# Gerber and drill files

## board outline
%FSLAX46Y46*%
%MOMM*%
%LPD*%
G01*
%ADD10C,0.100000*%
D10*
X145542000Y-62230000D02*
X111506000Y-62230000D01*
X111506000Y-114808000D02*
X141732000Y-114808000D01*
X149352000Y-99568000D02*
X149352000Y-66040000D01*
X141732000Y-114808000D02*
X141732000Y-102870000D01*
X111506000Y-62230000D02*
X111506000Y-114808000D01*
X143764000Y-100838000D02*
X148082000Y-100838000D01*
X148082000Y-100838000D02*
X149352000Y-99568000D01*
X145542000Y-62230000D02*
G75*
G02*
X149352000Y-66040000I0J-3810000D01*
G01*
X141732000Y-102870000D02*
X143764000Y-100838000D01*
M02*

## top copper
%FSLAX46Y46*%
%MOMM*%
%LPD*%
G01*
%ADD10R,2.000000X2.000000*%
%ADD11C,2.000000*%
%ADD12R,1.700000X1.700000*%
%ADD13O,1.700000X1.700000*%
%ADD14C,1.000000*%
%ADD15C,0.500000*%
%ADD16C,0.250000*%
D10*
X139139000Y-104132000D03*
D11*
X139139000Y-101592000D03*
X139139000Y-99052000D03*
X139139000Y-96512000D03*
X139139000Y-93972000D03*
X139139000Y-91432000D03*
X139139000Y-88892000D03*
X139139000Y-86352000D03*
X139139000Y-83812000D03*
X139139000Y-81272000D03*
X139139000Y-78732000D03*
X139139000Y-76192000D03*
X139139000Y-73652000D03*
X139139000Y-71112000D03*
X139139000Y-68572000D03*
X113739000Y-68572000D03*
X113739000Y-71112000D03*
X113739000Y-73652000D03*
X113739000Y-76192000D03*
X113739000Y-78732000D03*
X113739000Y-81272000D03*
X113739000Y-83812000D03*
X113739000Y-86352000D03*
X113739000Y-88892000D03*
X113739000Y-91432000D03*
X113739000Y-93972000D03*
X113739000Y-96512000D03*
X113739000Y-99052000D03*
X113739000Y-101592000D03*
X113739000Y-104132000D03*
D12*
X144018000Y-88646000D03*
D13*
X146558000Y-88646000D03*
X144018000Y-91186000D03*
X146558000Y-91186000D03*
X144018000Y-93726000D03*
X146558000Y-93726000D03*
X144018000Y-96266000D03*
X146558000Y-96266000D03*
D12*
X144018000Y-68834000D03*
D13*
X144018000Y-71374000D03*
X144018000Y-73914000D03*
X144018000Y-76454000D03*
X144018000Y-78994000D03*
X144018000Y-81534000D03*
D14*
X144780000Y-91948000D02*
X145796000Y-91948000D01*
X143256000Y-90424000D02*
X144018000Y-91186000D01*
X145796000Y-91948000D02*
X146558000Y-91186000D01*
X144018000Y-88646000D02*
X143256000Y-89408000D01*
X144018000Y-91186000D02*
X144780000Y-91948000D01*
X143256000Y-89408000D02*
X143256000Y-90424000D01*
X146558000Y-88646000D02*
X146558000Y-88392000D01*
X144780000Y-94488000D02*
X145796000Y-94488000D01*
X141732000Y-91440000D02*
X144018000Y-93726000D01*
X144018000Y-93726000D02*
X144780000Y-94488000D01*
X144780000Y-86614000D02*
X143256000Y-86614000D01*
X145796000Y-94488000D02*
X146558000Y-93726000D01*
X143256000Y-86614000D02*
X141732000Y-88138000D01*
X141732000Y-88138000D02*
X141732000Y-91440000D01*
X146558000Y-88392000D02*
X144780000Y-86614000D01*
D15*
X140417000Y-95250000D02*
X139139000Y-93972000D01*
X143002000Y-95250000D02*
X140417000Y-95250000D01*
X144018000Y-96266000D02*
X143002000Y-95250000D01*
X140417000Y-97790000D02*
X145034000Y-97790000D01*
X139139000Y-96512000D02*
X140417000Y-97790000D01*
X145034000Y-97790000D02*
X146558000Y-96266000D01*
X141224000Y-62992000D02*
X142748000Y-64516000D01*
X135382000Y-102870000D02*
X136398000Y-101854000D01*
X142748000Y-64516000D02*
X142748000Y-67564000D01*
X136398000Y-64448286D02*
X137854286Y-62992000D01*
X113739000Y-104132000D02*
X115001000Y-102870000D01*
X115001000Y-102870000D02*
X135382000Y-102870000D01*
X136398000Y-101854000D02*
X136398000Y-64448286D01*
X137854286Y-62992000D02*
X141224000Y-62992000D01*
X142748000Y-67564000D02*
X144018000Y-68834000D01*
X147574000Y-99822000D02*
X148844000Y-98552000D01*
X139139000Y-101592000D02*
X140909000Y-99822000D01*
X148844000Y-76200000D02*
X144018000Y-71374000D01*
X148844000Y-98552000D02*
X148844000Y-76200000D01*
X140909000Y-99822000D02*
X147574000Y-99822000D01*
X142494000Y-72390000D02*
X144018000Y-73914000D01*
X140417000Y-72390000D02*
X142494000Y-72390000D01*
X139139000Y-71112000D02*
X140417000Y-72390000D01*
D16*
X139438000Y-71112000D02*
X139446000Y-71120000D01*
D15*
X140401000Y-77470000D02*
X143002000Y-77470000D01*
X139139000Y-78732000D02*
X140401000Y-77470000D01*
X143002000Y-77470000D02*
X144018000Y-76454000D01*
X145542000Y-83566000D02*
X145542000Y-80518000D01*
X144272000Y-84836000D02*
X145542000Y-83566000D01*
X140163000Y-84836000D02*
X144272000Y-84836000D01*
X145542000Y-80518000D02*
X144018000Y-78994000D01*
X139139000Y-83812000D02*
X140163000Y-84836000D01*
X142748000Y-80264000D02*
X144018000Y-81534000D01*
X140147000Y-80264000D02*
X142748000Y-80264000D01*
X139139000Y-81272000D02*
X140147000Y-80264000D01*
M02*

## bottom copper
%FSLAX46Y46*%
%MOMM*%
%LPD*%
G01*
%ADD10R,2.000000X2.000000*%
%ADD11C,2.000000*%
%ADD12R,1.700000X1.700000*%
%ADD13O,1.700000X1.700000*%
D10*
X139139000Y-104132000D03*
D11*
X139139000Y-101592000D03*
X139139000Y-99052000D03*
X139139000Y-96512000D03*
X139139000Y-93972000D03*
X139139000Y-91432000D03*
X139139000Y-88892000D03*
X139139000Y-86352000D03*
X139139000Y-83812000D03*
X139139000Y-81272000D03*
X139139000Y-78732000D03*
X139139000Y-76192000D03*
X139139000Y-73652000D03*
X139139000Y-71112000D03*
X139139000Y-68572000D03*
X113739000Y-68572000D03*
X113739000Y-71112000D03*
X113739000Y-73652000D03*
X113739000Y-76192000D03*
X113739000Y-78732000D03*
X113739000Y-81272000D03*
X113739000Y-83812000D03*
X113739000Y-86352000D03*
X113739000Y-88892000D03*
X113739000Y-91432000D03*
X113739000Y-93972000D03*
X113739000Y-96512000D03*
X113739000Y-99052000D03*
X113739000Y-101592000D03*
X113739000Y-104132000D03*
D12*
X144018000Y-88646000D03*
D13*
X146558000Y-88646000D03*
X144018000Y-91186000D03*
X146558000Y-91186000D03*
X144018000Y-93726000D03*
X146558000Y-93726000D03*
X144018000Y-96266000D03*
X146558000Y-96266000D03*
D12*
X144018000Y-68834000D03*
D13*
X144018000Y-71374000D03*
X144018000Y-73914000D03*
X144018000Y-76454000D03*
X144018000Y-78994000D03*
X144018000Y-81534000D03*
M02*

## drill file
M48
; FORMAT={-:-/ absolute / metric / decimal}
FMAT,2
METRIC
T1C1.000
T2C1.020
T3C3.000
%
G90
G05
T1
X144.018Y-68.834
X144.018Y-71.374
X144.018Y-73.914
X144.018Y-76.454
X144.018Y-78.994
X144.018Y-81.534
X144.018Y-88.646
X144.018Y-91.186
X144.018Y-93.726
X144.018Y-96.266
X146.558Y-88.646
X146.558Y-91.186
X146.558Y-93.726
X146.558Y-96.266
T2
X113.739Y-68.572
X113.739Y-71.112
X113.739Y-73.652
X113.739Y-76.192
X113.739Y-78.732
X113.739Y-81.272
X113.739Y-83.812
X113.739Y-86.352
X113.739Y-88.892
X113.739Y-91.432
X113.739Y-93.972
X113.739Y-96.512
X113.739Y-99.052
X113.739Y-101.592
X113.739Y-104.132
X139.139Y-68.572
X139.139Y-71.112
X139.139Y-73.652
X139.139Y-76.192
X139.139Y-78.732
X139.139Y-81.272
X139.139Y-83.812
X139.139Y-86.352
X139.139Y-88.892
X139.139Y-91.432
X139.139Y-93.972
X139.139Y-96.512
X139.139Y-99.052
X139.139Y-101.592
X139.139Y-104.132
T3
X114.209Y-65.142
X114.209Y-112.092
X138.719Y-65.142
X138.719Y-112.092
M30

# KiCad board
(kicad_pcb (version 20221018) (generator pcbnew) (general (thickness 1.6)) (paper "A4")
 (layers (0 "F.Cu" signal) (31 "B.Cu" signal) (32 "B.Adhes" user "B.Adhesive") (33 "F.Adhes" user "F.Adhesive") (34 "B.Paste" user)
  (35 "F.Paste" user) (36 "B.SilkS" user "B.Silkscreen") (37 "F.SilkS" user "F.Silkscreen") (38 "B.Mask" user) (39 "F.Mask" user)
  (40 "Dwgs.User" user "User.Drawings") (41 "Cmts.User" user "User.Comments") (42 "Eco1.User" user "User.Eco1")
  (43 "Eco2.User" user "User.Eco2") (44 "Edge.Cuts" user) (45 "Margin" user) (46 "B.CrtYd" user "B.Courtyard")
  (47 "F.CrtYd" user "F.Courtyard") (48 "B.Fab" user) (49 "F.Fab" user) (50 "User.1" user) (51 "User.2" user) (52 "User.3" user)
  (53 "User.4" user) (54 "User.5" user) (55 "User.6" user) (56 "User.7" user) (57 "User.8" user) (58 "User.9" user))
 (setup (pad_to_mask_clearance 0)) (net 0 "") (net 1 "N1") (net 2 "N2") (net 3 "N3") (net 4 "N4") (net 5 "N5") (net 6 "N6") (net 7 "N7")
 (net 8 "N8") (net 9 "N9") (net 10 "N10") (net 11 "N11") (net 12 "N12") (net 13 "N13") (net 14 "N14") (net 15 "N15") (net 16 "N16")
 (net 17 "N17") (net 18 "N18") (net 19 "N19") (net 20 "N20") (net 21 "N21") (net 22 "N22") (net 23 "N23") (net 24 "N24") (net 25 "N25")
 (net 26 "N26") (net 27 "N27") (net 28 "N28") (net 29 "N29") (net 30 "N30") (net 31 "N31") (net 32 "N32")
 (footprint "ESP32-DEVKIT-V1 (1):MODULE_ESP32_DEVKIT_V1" (layer "F.Cu") (at 126.439 88.617 180)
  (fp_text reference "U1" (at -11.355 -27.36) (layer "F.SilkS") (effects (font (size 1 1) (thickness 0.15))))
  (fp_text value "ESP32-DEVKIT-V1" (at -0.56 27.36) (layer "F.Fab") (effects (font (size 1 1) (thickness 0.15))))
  (pad "" np_thru_hole circle (at -12.28 -23.475 180) (size 3 3) (drill 3) (layers "*.Cu" "*.Mask"))
  (pad "" np_thru_hole circle (at -12.28 23.475 180) (size 3 3) (drill 3) (layers "*.Cu" "*.Mask"))
  (pad "" np_thru_hole circle (at 12.23 -23.475 180) (size 3 3) (drill 3) (layers "*.Cu" "*.Mask"))
  (pad "" np_thru_hole circle (at 12.23 23.475 180) (size 3 3) (drill 3) (layers "*.Cu" "*.Mask"))
  (pad "1" thru_hole rect (at -12.7 -15.515 180) (size 2 2) (drill 1.02) (layers "*.Cu" "*.Mask") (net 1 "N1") (solder_mask_margin 0.102))
  (pad "2" thru_hole circle (at -12.7 -12.975 180) (size 2 2) (drill 1.02) (layers "*.Cu" "*.Mask") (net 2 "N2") (solder_mask_margin 0.102))
  (pad "3" thru_hole circle (at -12.7 -10.435 180) (size 2 2) (drill 1.02) (layers "*.Cu" "*.Mask") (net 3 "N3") (solder_mask_margin 0.102))
  (pad "4" thru_hole circle (at -12.7 -7.895 180) (size 2 2) (drill 1.02) (layers "*.Cu" "*.Mask") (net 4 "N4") (solder_mask_margin 0.102))
  (pad "5" thru_hole circle (at -12.7 -5.355 180) (size 2 2) (drill 1.02) (layers "*.Cu" "*.Mask") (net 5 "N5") (solder_mask_margin 0.102))
  (pad "6" thru_hole circle (at -12.7 -2.815 180) (size 2 2) (drill 1.02) (layers "*.Cu" "*.Mask") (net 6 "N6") (solder_mask_margin 0.102))
  (pad "7" thru_hole circle (at -12.7 -0.275 180) (size 2 2) (drill 1.02) (layers "*.Cu" "*.Mask") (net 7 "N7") (solder_mask_margin 0.102))
  (pad "8" thru_hole circle (at -12.7 2.265 180) (size 2 2) (drill 1.02) (layers "*.Cu" "*.Mask") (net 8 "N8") (solder_mask_margin 0.102))
  (pad "9" thru_hole circle (at -12.7 4.805 180) (size 2 2) (drill 1.02) (layers "*.Cu" "*.Mask") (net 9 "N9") (solder_mask_margin 0.102))
  (pad "10" thru_hole circle (at -12.7 7.345 180) (size 2 2) (drill 1.02) (layers "*.Cu" "*.Mask") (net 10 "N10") (solder_mask_margin 0.102))
  (pad "11" thru_hole circle (at -12.7 9.885 180) (size 2 2) (drill 1.02) (layers "*.Cu" "*.Mask") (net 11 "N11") (solder_mask_margin 0.102))
  (pad "12" thru_hole circle (at -12.7 12.425 180) (size 2 2) (drill 1.02) (layers "*.Cu" "*.Mask") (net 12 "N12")
   (solder_mask_margin 0.102))
  (pad "13" thru_hole circle (at -12.7 14.965 180) (size 2 2) (drill 1.02) (layers "*.Cu" "*.Mask") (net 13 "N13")
   (solder_mask_margin 0.102))
  (pad "14" thru_hole circle (at -12.7 17.505 180) (size 2 2) (drill 1.02) (layers "*.Cu" "*.Mask") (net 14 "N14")
   (solder_mask_margin 0.102))
  (pad "15" thru_hole circle (at -12.7 20.045 180) (size 2 2) (drill 1.02) (layers "*.Cu" "*.Mask") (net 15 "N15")
   (solder_mask_margin 0.102))
  (pad "16" thru_hole circle (at 12.7 20.045 180) (size 2 2) (drill 1.02) (layers "*.Cu" "*.Mask") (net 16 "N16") (solder_mask_margin 0.102))
  (pad "17" thru_hole circle (at 12.7 17.505 180) (size 2 2) (drill 1.02) (layers "*.Cu" "*.Mask") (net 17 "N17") (solder_mask_margin 0.102))
  (pad "18" thru_hole circle (at 12.7 14.965 180) (size 2 2) (drill 1.02) (layers "*.Cu" "*.Mask") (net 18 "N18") (solder_mask_margin 0.102))
  (pad "19" thru_hole circle (at 12.7 12.425 180) (size 2 2) (drill 1.02) (layers "*.Cu" "*.Mask") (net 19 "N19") (solder_mask_margin 0.102))
  (pad "20" thru_hole circle (at 12.7 9.885 180) (size 2 2) (drill 1.02) (layers "*.Cu" "*.Mask") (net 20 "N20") (solder_mask_margin 0.102))
  (pad "21" thru_hole circle (at 12.7 7.345 180) (size 2 2) (drill 1.02) (layers "*.Cu" "*.Mask") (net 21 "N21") (solder_mask_margin 0.102))
  (pad "22" thru_hole circle (at 12.7 4.805 180) (size 2 2) (drill 1.02) (layers "*.Cu" "*.Mask") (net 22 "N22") (solder_mask_margin 0.102))
  (pad "23" thru_hole circle (at 12.7 2.265 180) (size 2 2) (drill 1.02) (layers "*.Cu" "*.Mask") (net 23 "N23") (solder_mask_margin 0.102))
  (pad "24" thru_hole circle (at 12.7 -0.275 180) (size 2 2) (drill 1.02) (layers "*.Cu" "*.Mask") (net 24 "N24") (solder_mask_margin 0.102))
  (pad "25" thru_hole circle (at 12.7 -2.815 180) (size 2 2) (drill 1.02) (layers "*.Cu" "*.Mask") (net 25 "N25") (solder_mask_margin 0.102))
  (pad "26" thru_hole circle (at 12.7 -5.355 180) (size 2 2) (drill 1.02) (layers "*.Cu" "*.Mask") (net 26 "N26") (solder_mask_margin 0.102))
  (pad "27" thru_hole circle (at 12.7 -7.895 180) (size 2 2) (drill 1.02) (layers "*.Cu" "*.Mask") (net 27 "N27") (solder_mask_margin 0.102))
  (pad "28" thru_hole circle (at 12.7 -10.435 180) (size 2 2) (drill 1.02) (layers "*.Cu" "*.Mask") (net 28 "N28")
   (solder_mask_margin 0.102))
  (pad "29" thru_hole circle (at 12.7 -12.975 180) (size 2 2) (drill 1.02) (layers "*.Cu" "*.Mask") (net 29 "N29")
   (solder_mask_margin 0.102))
  (pad "30" thru_hole circle (at 12.7 -15.515 180) (size 2 2) (drill 1.02) (layers "*.Cu" "*.Mask") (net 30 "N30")
   (solder_mask_margin 0.102))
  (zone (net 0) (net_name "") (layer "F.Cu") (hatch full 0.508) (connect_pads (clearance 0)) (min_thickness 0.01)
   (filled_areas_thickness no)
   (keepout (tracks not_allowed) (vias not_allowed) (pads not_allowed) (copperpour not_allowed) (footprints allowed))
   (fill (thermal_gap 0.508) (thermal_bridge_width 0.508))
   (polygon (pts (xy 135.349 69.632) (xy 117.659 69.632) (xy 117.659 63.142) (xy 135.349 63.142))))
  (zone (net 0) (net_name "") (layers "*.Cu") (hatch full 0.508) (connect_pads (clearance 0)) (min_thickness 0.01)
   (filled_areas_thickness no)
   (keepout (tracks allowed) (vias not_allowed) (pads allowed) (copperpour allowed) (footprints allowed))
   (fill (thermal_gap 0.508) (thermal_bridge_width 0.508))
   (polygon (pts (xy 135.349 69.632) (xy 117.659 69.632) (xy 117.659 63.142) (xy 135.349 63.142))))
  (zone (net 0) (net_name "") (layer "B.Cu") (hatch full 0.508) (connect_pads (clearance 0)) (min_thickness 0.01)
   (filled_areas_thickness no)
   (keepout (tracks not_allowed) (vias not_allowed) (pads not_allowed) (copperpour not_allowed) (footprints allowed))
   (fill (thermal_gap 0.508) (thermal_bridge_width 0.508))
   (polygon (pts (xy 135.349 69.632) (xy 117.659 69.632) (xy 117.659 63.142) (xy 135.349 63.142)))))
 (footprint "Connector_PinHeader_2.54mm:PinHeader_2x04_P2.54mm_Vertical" (layer "F.Cu") (at 144.018 88.646)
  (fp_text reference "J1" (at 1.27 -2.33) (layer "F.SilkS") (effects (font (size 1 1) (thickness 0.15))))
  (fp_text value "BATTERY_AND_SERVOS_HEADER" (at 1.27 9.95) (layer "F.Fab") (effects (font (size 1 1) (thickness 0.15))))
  (pad "1" thru_hole rect (at 0 0) (size 1.7 1.7) (drill 1) (layers "*.Cu" "*.Mask") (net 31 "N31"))
  (pad "2" thru_hole oval (at 2.54 0) (size 1.7 1.7) (drill 1) (layers "*.Cu" "*.Mask") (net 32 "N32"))
  (pad "3" thru_hole oval (at 0 2.54) (size 1.7 1.7) (drill 1) (layers "*.Cu" "*.Mask") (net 31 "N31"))
  (pad "4" thru_hole oval (at 2.54 2.54) (size 1.7 1.7) (drill 1) (layers "*.Cu" "*.Mask") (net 31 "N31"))
  (pad "5" thru_hole oval (at 0 5.08) (size 1.7 1.7) (drill 1) (layers "*.Cu" "*.Mask") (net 32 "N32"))
  (pad "6" thru_hole oval (at 2.54 5.08) (size 1.7 1.7) (drill 1) (layers "*.Cu" "*.Mask") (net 32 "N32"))
  (pad "7" thru_hole oval (at 0 7.62) (size 1.7 1.7) (drill 1) (layers "*.Cu" "*.Mask") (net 5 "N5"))
  (pad "8" thru_hole oval (at 2.54 7.62) (size 1.7 1.7) (drill 1) (layers "*.Cu" "*.Mask") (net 4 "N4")))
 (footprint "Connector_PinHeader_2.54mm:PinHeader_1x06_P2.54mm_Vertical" (layer "F.Cu") (at 144.018 68.834)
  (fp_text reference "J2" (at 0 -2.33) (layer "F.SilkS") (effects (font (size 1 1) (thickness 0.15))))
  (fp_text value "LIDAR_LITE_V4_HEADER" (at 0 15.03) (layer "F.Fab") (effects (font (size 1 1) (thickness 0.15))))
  (pad "1" thru_hole rect (at 0 0) (size 1.7 1.7) (drill 1) (layers "*.Cu" "*.Mask") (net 30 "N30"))
  (pad "2" thru_hole oval (at 0 2.54) (size 1.7 1.7) (drill 1) (layers "*.Cu" "*.Mask") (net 2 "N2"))
  (pad "3" thru_hole oval (at 0 5.08) (size 1.7 1.7) (drill 1) (layers "*.Cu" "*.Mask") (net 14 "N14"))
  (pad "4" thru_hole oval (at 0 7.62) (size 1.7 1.7) (drill 1) (layers "*.Cu" "*.Mask") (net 11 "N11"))
  (pad "5" thru_hole oval (at 0 10.16) (size 1.7 1.7) (drill 1) (layers "*.Cu" "*.Mask") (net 9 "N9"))
  (pad "6" thru_hole oval (at 0 12.7) (size 1.7 1.7) (drill 1) (layers "*.Cu" "*.Mask") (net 10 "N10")))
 (gr_line (start 145.542 62.23) (end 111.506 62.23) (stroke (width 0.1) (type default)) (layer "Edge.Cuts"))
 (gr_line (start 111.506 114.808) (end 141.732 114.808) (stroke (width 0.1) (type default)) (layer "Edge.Cuts"))
 (gr_line (start 149.352 99.568) (end 149.352 66.04) (stroke (width 0.1) (type default)) (layer "Edge.Cuts"))
 (gr_line (start 141.732 114.808) (end 141.732 102.87) (stroke (width 0.1) (type default)) (layer "Edge.Cuts"))
 (gr_line (start 111.506 62.23) (end 111.506 114.808) (stroke (width 0.1) (type default)) (layer "Edge.Cuts"))
 (gr_line (start 143.764 100.838) (end 148.082 100.838) (stroke (width 0.1) (type default)) (layer "Edge.Cuts"))
 (gr_line (start 148.082 100.838) (end 149.352 99.568) (stroke (width 0.1) (type default)) (layer "Edge.Cuts"))
 (gr_arc (start 145.542 62.23) (mid 148.236077 63.345923) (end 149.352 66.04) (stroke (width 0.1) (type default)) (layer "Edge.Cuts"))
 (gr_line (start 141.732 102.87) (end 143.764 100.838) (stroke (width 0.1) (type default)) (layer "Edge.Cuts"))
 (segment (start 144.78 91.948) (end 145.796 91.948) (width 1) (layer "F.Cu") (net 31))
 (segment (start 143.256 90.424) (end 144.018 91.186) (width 1) (layer "F.Cu") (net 31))
 (segment (start 145.796 91.948) (end 146.558 91.186) (width 1) (layer "F.Cu") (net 31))
 (segment (start 144.018 88.646) (end 143.256 89.408) (width 1) (layer "F.Cu") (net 31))
 (segment (start 144.018 91.186) (end 144.78 91.948) (width 1) (layer "F.Cu") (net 31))
 (segment (start 143.256 89.408) (end 143.256 90.424) (width 1) (layer "F.Cu") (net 31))
 (segment (start 146.558 88.646) (end 146.558 88.392) (width 1) (layer "F.Cu") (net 32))
 (segment (start 144.78 94.488) (end 145.796 94.488) (width 1) (layer "F.Cu") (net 32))
 (segment (start 141.732 91.44) (end 144.018 93.726) (width 1) (layer "F.Cu") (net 32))
 (segment (start 144.018 93.726) (end 144.78 94.488) (width 1) (layer "F.Cu") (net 32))
 (segment (start 144.78 86.614) (end 143.256 86.614) (width 1) (layer "F.Cu") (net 32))
 (segment (start 145.796 94.488) (end 146.558 93.726) (width 1) (layer "F.Cu") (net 32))
 (segment (start 143.256 86.614) (end 141.732 88.138) (width 1) (layer "F.Cu") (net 32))
 (segment (start 141.732 88.138) (end 141.732 91.44) (width 1) (layer "F.Cu") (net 32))
 (segment (start 146.558 88.392) (end 144.78 86.614) (width 1) (layer "F.Cu") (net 32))
 (segment (start 140.417 95.25) (end 139.139 93.972) (width 0.5) (layer "F.Cu") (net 5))
 (segment (start 143.002 95.25) (end 140.417 95.25) (width 0.5) (layer "F.Cu") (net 5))
 (segment (start 144.018 96.266) (end 143.002 95.25) (width 0.5) (layer "F.Cu") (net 5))
 (segment (start 140.417 97.79) (end 145.034 97.79) (width 0.5) (layer "F.Cu") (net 4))
 (segment (start 139.139 96.512) (end 140.417 97.79) (width 0.5) (layer "F.Cu") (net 4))
 (segment (start 145.034 97.79) (end 146.558 96.266) (width 0.5) (layer "F.Cu") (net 4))
 (segment (start 141.224 62.992) (end 142.748 64.516) (width 0.5) (layer "F.Cu") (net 30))
 (segment (start 135.382 102.87) (end 136.398 101.854) (width 0.5) (layer "F.Cu") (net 30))
 (segment (start 142.748 64.516) (end 142.748 67.564) (width 0.5) (layer "F.Cu") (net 30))
 (segment (start 136.398 64.448286) (end 137.854286 62.992) (width 0.5) (layer "F.Cu") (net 30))
 (segment (start 113.739 104.132) (end 115.001 102.87) (width 0.5) (layer "F.Cu") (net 30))
 (segment (start 115.001 102.87) (end 135.382 102.87) (width 0.5) (layer "F.Cu") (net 30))
 (segment (start 136.398 101.854) (end 136.398 64.448286) (width 0.5) (layer "F.Cu") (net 30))
 (segment (start 137.854286 62.992) (end 141.224 62.992) (width 0.5) (layer "F.Cu") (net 30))
 (segment (start 142.748 67.564) (end 144.018 68.834) (width 0.5) (layer "F.Cu") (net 30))
 (segment (start 147.574 99.822) (end 148.844 98.552) (width 0.5) (layer "F.Cu") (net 2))
 (segment (start 139.139 101.592) (end 140.909 99.822) (width 0.5) (layer "F.Cu") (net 2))
 (segment (start 148.844 76.2) (end 144.018 71.374) (width 0.5) (layer "F.Cu") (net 2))
 (segment (start 148.844 98.552) (end 148.844 76.2) (width 0.5) (layer "F.Cu") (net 2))
 (segment (start 140.909 99.822) (end 147.574 99.822) (width 0.5) (layer "F.Cu") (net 2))
 (segment (start 142.494 72.39) (end 144.018 73.914) (width 0.5) (layer "F.Cu") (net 14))
 (segment (start 140.417 72.39) (end 142.494 72.39) (width 0.5) (layer "F.Cu") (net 14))
 (segment (start 139.139 71.112) (end 140.417 72.39) (width 0.5) (layer "F.Cu") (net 14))
 (segment (start 139.438 71.112) (end 139.446 71.12) (width 0.25) (layer "F.Cu") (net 14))
 (segment (start 140.401 77.47) (end 143.002 77.47) (width 0.5) (layer "F.Cu") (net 11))
 (segment (start 139.139 78.732) (end 140.401 77.47) (width 0.5) (layer "F.Cu") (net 11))
 (segment (start 143.002 77.47) (end 144.018 76.454) (width 0.5) (layer "F.Cu") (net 11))
 (segment (start 145.542 83.566) (end 145.542 80.518) (width 0.5) (layer "F.Cu") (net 9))
 (segment (start 144.272 84.836) (end 145.542 83.566) (width 0.5) (layer "F.Cu") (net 9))
 (segment (start 140.163 84.836) (end 144.272 84.836) (width 0.5) (layer "F.Cu") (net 9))
 (segment (start 145.542 80.518) (end 144.018 78.994) (width 0.5) (layer "F.Cu") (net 9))
 (segment (start 139.139 83.812) (end 140.163 84.836) (width 0.5) (layer "F.Cu") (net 9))
 (segment (start 142.748 80.264) (end 144.018 81.534) (width 0.5) (layer "F.Cu") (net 10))
 (segment (start 140.147 80.264) (end 142.748 80.264) (width 0.5) (layer "F.Cu") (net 10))
 (segment (start 139.139 81.272) (end 140.147 80.264) (width 0.5) (layer "F.Cu") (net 10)))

